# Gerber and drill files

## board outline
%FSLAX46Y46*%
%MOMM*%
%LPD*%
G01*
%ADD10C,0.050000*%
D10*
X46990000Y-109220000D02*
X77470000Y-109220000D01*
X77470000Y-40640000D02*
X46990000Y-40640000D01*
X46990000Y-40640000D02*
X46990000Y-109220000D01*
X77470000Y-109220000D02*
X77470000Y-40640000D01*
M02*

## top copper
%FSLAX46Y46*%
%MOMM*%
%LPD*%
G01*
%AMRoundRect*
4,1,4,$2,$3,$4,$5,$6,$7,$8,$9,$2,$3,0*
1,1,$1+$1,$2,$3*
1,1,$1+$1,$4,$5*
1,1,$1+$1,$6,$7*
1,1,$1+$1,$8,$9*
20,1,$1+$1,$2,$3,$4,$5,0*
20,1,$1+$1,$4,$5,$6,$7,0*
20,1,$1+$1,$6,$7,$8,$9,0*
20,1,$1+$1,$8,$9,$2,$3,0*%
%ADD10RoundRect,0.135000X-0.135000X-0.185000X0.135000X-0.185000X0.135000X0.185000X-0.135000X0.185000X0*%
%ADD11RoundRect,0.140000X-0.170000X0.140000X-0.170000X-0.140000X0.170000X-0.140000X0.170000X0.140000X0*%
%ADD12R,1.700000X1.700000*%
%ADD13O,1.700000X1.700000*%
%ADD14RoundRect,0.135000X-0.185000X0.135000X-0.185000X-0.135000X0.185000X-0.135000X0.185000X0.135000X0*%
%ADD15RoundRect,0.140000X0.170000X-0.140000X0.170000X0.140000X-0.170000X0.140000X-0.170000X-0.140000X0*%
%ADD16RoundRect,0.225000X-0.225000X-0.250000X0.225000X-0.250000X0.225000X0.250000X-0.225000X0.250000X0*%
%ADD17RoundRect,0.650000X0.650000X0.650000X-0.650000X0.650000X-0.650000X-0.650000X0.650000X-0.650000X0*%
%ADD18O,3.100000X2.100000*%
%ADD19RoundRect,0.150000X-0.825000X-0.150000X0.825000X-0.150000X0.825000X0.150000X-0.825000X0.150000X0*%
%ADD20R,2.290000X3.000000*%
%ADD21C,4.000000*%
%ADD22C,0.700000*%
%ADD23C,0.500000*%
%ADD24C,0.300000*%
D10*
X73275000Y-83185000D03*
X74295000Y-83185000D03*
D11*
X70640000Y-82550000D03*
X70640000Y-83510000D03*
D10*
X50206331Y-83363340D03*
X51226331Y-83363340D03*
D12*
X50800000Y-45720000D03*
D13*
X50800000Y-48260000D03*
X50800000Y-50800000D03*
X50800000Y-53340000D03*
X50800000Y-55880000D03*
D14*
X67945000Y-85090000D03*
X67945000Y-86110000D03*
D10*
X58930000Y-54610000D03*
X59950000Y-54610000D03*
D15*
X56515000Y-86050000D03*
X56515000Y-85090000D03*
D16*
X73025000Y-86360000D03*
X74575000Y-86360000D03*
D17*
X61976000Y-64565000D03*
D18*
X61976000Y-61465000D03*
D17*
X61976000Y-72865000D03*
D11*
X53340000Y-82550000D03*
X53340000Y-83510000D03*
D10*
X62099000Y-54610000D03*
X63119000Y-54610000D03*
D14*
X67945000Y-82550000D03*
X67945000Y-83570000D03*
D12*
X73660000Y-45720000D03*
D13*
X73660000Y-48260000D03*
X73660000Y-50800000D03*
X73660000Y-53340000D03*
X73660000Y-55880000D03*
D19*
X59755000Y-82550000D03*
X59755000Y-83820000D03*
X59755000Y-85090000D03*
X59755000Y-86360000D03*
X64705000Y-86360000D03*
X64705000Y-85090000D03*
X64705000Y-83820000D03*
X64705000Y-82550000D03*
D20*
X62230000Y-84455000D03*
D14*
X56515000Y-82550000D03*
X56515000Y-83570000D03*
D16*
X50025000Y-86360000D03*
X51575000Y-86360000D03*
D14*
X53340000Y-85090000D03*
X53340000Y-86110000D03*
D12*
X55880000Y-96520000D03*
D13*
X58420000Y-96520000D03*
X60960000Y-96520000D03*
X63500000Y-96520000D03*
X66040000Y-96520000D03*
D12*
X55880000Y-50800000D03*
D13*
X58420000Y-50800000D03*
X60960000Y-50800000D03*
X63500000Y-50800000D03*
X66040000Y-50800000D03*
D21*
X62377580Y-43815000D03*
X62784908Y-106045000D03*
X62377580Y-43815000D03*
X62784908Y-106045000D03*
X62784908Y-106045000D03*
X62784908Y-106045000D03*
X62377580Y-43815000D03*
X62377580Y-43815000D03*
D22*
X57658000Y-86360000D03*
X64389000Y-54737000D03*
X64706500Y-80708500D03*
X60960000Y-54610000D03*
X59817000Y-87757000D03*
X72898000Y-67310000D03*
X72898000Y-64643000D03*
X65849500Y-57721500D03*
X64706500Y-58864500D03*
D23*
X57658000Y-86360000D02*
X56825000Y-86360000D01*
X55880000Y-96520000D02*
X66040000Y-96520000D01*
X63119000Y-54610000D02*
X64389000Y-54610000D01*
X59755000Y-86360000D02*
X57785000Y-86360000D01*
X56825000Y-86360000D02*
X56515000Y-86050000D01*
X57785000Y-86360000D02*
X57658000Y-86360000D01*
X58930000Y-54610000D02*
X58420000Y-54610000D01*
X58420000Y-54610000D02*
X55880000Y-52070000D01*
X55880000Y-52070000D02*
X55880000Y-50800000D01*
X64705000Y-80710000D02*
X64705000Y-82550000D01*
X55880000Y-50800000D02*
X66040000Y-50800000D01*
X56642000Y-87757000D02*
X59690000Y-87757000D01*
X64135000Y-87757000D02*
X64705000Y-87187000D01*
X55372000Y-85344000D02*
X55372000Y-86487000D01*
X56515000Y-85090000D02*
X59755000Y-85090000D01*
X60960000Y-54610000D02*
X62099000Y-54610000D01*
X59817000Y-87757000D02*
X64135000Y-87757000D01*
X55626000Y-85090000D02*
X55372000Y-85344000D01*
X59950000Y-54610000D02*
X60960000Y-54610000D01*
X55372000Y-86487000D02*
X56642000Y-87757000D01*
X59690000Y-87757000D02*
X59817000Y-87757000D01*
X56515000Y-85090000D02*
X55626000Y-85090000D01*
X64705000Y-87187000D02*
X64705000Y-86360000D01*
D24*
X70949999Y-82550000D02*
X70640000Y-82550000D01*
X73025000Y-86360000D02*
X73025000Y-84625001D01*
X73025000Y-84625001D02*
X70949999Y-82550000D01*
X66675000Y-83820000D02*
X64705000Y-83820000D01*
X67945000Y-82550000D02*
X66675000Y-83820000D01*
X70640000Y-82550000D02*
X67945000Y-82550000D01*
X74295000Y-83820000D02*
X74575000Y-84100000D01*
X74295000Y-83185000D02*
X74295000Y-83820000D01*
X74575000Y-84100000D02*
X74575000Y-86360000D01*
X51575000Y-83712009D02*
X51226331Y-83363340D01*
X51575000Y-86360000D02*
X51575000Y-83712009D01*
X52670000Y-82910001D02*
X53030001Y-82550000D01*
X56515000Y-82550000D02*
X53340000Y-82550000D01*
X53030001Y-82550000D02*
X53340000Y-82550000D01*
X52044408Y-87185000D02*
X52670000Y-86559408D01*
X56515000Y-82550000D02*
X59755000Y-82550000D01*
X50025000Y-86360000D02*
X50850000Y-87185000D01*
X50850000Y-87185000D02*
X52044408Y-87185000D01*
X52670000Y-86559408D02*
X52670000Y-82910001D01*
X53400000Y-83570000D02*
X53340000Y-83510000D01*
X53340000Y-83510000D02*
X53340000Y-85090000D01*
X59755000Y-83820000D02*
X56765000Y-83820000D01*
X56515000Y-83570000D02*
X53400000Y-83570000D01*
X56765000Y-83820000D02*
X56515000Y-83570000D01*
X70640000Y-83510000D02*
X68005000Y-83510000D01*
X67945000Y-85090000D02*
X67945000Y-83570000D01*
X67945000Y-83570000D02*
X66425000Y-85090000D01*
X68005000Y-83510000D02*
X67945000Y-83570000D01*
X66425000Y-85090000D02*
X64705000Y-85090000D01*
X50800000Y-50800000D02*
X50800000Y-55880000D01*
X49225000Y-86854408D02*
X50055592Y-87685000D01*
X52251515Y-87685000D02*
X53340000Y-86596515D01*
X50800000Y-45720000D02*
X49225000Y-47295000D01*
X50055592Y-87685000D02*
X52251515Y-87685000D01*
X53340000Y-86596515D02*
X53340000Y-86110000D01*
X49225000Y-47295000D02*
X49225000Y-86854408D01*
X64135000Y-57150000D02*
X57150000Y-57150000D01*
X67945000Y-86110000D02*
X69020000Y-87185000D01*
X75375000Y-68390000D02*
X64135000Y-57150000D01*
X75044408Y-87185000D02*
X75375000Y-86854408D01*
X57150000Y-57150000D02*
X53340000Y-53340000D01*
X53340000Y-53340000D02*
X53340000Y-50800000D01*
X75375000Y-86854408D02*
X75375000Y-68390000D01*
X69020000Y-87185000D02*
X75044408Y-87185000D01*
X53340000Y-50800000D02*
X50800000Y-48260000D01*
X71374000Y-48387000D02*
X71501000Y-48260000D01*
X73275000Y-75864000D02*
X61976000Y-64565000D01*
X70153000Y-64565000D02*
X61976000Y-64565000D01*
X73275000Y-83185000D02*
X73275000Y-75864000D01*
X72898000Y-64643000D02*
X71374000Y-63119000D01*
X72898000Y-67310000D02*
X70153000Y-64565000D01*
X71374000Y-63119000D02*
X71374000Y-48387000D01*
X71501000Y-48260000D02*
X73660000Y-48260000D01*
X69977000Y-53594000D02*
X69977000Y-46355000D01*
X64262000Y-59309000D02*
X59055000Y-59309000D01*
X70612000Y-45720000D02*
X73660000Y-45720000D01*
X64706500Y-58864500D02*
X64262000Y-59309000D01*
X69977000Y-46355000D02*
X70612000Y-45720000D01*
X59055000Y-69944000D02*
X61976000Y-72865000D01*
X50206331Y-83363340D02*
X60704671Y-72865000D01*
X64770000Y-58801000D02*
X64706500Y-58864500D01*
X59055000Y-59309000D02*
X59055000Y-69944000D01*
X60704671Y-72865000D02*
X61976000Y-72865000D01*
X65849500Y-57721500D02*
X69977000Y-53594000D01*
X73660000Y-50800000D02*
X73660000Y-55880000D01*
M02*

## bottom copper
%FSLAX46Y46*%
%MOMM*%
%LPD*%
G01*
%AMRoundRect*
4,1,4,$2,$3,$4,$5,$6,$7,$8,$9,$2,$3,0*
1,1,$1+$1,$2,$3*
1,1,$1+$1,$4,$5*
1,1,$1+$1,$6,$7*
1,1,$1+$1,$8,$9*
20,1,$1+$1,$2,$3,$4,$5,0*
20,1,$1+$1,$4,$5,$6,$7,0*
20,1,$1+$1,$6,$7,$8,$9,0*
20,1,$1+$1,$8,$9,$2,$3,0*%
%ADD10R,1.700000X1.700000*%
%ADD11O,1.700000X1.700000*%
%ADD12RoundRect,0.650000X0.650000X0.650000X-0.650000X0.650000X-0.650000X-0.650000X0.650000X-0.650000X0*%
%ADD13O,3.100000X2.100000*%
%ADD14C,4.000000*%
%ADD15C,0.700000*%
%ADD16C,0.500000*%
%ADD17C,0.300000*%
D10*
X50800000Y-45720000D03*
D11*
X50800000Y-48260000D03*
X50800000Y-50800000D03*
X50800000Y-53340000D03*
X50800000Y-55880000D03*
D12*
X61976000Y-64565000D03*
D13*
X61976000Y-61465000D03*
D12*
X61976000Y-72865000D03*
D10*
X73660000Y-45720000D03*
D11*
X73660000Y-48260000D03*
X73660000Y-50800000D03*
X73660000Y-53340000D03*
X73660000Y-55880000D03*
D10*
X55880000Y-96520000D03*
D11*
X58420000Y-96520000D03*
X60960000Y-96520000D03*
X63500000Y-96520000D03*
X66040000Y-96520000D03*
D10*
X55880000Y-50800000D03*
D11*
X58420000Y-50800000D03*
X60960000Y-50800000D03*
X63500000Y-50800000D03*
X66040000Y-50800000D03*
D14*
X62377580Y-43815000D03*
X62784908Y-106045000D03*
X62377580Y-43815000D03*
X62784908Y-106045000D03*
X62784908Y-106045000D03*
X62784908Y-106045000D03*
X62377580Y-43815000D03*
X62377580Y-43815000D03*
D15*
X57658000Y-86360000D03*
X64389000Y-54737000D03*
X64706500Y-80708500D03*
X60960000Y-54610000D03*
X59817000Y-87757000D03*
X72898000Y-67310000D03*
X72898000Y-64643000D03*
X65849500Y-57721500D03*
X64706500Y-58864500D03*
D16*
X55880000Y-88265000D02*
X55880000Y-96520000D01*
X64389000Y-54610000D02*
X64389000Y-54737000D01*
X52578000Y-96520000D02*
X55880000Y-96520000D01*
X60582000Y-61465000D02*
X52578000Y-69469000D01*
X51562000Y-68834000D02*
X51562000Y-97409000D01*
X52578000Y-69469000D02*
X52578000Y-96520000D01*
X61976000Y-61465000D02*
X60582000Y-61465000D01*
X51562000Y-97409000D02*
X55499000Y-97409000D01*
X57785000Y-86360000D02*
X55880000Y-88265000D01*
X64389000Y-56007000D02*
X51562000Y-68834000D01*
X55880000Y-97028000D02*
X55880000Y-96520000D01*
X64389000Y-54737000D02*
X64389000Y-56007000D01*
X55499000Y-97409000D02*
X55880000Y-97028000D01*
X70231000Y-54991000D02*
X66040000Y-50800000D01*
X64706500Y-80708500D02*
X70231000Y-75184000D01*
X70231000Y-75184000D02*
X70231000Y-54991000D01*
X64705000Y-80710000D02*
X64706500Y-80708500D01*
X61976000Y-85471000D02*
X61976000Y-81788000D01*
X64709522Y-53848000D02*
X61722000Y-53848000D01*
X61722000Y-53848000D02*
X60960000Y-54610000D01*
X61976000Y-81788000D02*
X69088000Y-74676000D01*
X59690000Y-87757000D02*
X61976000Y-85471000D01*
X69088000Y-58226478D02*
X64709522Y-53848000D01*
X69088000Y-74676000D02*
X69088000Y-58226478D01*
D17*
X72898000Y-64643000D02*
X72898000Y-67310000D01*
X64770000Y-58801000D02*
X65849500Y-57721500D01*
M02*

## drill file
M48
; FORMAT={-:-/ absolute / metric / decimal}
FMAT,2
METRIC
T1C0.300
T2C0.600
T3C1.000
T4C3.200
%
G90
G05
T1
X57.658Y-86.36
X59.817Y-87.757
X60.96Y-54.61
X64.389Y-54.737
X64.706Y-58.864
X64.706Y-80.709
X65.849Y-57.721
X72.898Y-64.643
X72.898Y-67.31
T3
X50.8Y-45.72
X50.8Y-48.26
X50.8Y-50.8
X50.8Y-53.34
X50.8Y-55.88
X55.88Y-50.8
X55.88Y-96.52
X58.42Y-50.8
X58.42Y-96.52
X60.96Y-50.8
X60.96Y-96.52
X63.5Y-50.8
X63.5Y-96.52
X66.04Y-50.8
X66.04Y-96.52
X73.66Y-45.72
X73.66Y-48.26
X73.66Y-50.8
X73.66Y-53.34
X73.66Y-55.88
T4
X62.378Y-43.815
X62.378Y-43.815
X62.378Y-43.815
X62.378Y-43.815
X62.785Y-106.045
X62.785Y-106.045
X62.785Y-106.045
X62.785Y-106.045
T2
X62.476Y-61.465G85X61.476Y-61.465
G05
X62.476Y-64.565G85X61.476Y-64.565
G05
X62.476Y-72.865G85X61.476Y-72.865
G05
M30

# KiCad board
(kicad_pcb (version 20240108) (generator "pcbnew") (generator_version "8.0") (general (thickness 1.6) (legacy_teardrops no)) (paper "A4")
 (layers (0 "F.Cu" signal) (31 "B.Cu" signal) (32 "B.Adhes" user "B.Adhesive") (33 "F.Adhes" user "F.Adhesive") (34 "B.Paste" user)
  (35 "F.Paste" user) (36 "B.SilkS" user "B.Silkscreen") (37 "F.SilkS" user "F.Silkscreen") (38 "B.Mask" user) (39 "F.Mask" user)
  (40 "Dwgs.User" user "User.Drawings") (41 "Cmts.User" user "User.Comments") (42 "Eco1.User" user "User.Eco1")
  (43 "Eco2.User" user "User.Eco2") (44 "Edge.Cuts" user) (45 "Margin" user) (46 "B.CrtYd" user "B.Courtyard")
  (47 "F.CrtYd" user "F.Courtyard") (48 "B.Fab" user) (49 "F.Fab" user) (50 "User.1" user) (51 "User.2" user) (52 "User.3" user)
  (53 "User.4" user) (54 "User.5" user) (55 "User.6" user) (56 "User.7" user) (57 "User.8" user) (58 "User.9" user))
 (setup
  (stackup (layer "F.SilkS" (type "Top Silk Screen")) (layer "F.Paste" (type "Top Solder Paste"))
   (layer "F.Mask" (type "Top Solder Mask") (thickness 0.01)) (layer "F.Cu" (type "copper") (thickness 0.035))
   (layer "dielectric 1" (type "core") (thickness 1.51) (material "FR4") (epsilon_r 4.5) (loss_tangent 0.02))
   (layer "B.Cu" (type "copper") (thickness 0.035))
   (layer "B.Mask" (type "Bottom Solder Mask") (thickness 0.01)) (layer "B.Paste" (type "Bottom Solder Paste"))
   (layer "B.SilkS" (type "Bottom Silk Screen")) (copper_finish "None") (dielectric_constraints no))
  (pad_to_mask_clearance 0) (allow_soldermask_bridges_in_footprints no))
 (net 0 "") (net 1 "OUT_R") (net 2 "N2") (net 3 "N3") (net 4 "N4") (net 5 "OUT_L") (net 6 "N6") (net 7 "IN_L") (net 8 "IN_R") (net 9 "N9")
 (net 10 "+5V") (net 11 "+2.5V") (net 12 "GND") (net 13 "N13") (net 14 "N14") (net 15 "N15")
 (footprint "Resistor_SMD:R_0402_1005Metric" (layer "F.Cu") (at 73.785 83.185)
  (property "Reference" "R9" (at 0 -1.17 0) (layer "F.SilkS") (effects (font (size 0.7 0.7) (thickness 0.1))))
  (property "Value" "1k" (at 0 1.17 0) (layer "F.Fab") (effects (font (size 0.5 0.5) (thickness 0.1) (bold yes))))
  (pad "1" smd roundrect (at -0.51 0) (size 0.54 0.64) (layers "F.Cu" "F.Paste" "F.Mask") (roundrect_rratio 0.25) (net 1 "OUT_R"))
  (pad "2" smd roundrect (at 0.51 0) (size 0.54 0.64) (layers "F.Cu" "F.Paste" "F.Mask") (roundrect_rratio 0.25) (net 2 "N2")))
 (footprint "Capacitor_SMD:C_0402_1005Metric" (layer "F.Cu") (at 70.64 83.03 -90)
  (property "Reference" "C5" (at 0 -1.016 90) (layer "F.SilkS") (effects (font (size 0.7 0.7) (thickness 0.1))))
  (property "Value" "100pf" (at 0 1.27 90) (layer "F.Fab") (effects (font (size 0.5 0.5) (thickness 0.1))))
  (pad "1" smd roundrect (at -0.48 0 270) (size 0.56 0.62) (layers "F.Cu" "F.Paste" "F.Mask") (roundrect_rratio 0.25) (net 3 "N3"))
  (pad "2" smd roundrect (at 0.48 0 270) (size 0.56 0.62) (layers "F.Cu" "F.Paste" "F.Mask") (roundrect_rratio 0.25) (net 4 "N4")))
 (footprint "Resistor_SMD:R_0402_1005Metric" (layer "F.Cu") (at 50.716331 83.36334)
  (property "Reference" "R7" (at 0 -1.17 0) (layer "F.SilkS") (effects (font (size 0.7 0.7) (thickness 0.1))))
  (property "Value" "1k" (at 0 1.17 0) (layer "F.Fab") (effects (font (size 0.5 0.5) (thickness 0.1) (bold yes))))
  (pad "1" smd roundrect (at -0.51 0) (size 0.54 0.64) (layers "F.Cu" "F.Paste" "F.Mask") (roundrect_rratio 0.25) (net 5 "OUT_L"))
  (pad "2" smd roundrect (at 0.51 0) (size 0.54 0.64) (layers "F.Cu" "F.Paste" "F.Mask") (roundrect_rratio 0.25) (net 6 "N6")))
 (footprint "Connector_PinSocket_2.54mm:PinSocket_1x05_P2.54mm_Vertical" (layer "F.Cu") (at 50.8 45.72)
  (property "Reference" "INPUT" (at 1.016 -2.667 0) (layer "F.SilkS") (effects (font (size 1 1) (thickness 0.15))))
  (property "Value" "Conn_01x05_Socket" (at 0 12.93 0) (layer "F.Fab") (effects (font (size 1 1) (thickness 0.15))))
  (pad "1" thru_hole rect (at 0 0) (size 1.7 1.7) (drill 1) (layers "*.Cu" "*.Mask") (remove_unused_layers no) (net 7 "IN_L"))
  (pad "2" thru_hole oval (at 0 2.54) (size 1.7 1.7) (drill 1) (layers "*.Cu" "*.Mask") (remove_unused_layers no) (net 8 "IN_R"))
  (pad "3" thru_hole oval (at 0 5.08) (size 1.7 1.7) (drill 1) (layers "*.Cu" "*.Mask") (remove_unused_layers no) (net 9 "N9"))
  (pad "4" thru_hole oval (at 0 7.62) (size 1.7 1.7) (drill 1) (layers "*.Cu" "*.Mask") (remove_unused_layers no) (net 9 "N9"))
  (pad "5" thru_hole oval (at 0 10.16) (size 1.7 1.7) (drill 1) (layers "*.Cu" "*.Mask") (remove_unused_layers no) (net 9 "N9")))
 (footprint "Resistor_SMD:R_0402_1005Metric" (layer "F.Cu") (at 67.945 85.6 -90)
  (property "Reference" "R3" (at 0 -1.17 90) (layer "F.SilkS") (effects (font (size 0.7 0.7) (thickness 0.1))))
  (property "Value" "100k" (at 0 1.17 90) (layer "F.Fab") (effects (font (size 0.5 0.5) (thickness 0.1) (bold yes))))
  (pad "1" smd roundrect (at -0.51 0 270) (size 0.54 0.64) (layers "F.Cu" "F.Paste" "F.Mask") (roundrect_rratio 0.25) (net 4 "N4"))
  (pad "2" smd roundrect (at 0.51 0 270) (size 0.54 0.64) (layers "F.Cu" "F.Paste" "F.Mask") (roundrect_rratio 0.25) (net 8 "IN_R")))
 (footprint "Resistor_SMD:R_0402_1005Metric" (layer "F.Cu") (at 59.44 54.61)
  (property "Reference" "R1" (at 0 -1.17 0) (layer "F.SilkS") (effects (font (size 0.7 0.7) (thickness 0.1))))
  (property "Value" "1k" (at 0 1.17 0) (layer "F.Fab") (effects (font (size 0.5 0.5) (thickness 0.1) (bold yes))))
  (pad "1" smd roundrect (at -0.51 0) (size 0.54 0.64) (layers "F.Cu" "F.Paste" "F.Mask") (roundrect_rratio 0.25) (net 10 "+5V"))
  (pad "2" smd roundrect (at 0.51 0) (size 0.54 0.64) (layers "F.Cu" "F.Paste" "F.Mask") (roundrect_rratio 0.25) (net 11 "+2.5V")))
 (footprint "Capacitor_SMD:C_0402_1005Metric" (layer "F.Cu") (at 56.515 85.57 90)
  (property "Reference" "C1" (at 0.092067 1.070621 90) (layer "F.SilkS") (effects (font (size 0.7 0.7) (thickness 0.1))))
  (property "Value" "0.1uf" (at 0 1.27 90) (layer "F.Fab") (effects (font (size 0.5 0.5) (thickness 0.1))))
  (pad "1" smd roundrect (at -0.48 0 90) (size 0.56 0.62) (layers "F.Cu" "F.Paste" "F.Mask") (roundrect_rratio 0.25) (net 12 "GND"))
  (pad "2" smd roundrect (at 0.48 0 90) (size 0.56 0.62) (layers "F.Cu" "F.Paste" "F.Mask") (roundrect_rratio 0.25) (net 11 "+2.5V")))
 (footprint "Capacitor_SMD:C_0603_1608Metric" (layer "F.Cu") (at 73.8 86.36)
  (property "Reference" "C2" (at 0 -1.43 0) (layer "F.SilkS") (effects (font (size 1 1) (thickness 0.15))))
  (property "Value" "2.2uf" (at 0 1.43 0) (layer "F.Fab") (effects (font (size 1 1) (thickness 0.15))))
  (pad "1" smd roundrect (at -0.775 0) (size 0.9 0.95) (layers "F.Cu" "F.Paste" "F.Mask") (roundrect_rratio 0.25) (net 3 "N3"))
  (pad "2" smd roundrect (at 0.775 0) (size 0.9 0.95) (layers "F.Cu" "F.Paste" "F.Mask") (roundrect_rratio 0.25) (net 2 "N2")))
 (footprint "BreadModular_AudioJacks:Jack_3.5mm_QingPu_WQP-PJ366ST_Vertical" (layer "F.Cu") (at 61.976 67.945 180)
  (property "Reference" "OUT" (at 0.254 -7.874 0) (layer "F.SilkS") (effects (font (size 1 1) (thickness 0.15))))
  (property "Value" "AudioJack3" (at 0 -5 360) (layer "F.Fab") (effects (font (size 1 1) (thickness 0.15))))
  (pad "R" thru_hole roundrect (at 0 3.38 180) (size 2.6 2.6) (drill oval 1.6 0.6) (layers "*.Cu" "*.Mask") (remove_unused_layers no)
   (roundrect_rratio 0.25) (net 1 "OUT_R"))
  (pad "S" thru_hole oval (at 0 6.48 180) (size 3.1 2.1) (drill oval 1.6 0.6) (layers "*.Cu" "*.Mask") (remove_unused_layers no)
   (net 12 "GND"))
  (pad "T" thru_hole roundrect (at 0 -4.92 180) (size 2.6 2.6) (drill oval 1.6 0.6) (layers "*.Cu" "*.Mask") (remove_unused_layers no)
   (roundrect_rratio 0.25) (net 5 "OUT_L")))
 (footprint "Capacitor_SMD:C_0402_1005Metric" (layer "F.Cu") (at 53.34 83.03 -90)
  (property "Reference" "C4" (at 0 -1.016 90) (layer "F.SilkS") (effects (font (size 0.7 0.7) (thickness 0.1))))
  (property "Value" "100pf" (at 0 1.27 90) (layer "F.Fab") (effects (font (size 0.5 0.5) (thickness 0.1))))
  (pad "1" smd roundrect (at -0.48 0 270) (size 0.56 0.62) (layers "F.Cu" "F.Paste" "F.Mask") (roundrect_rratio 0.25) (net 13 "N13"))
  (pad "2" smd roundrect (at 0.48 0 270) (size 0.56 0.62) (layers "F.Cu" "F.Paste" "F.Mask") (roundrect_rratio 0.25) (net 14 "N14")))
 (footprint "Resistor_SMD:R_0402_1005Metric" (layer "F.Cu") (at 62.609 54.61)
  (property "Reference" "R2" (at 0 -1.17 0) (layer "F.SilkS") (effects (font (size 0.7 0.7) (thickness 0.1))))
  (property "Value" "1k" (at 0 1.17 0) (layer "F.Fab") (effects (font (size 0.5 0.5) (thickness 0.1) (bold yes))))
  (pad "1" smd roundrect (at -0.51 0) (size 0.54 0.64) (layers "F.Cu" "F.Paste" "F.Mask") (roundrect_rratio 0.25) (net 11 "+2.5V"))
  (pad "2" smd roundrect (at 0.51 0) (size 0.54 0.64) (layers "F.Cu" "F.Paste" "F.Mask") (roundrect_rratio 0.25) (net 12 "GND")))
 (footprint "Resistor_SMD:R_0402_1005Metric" (layer "F.Cu") (at 67.945 83.06 -90)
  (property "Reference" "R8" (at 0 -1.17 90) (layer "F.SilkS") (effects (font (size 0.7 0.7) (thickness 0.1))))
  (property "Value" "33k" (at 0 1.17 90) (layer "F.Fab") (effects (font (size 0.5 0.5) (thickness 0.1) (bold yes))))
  (pad "1" smd roundrect (at -0.51 0 270) (size 0.54 0.64) (layers "F.Cu" "F.Paste" "F.Mask") (roundrect_rratio 0.25) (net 3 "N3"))
  (pad "2" smd roundrect (at 0.51 0 270) (size 0.54 0.64) (layers "F.Cu" "F.Paste" "F.Mask") (roundrect_rratio 0.25) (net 4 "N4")))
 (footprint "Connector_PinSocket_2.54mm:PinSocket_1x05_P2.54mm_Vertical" (layer "F.Cu") (at 73.66 45.72)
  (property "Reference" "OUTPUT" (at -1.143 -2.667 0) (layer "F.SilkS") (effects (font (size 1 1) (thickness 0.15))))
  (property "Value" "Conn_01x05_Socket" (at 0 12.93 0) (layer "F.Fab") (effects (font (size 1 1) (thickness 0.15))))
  (pad "1" thru_hole rect (at 0 0) (size 1.7 1.7) (drill 1) (layers "*.Cu" "*.Mask") (remove_unused_layers no) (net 5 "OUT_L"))
  (pad "2" thru_hole oval (at 0 2.54) (size 1.7 1.7) (drill 1) (layers "*.Cu" "*.Mask") (remove_unused_layers no) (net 1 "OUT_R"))
  (pad "3" thru_hole oval (at 0 5.08) (size 1.7 1.7) (drill 1) (layers "*.Cu" "*.Mask") (remove_unused_layers no) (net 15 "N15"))
  (pad "4" thru_hole oval (at 0 7.62) (size 1.7 1.7) (drill 1) (layers "*.Cu" "*.Mask") (remove_unused_layers no) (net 15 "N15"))
  (pad "5" thru_hole oval (at 0 10.16) (size 1.7 1.7) (drill 1) (layers "*.Cu" "*.Mask") (remove_unused_layers no) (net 15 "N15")))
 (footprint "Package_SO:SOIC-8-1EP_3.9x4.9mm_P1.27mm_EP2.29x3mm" (layer "F.Cu") (at 62.23 84.455)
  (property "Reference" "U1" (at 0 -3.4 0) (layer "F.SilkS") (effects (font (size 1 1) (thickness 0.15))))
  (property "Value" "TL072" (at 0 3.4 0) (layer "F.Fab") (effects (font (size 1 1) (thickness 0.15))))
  (pad "" smd roundrect (at -0.57 -0.75) (size 0.92 1.21) (layers "F.Paste") (roundrect_rratio 0.25))
  (pad "" smd roundrect (at -0.57 0.75) (size 0.92 1.21) (layers "F.Paste") (roundrect_rratio 0.25))
  (pad "" smd roundrect (at 0.57 -0.75) (size 0.92 1.21) (layers "F.Paste") (roundrect_rratio 0.25))
  (pad "" smd roundrect (at 0.57 0.75) (size 0.92 1.21) (layers "F.Paste") (roundrect_rratio 0.25))
  (pad "1" smd roundrect (at -2.475 -1.905) (size 1.95 0.6) (layers "F.Cu" "F.Paste" "F.Mask") (roundrect_rratio 0.25) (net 13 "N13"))
  (pad "2" smd roundrect (at -2.475 -0.635) (size 1.95 0.6) (layers "F.Cu" "F.Paste" "F.Mask") (roundrect_rratio 0.25) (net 14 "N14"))
  (pad "3" smd roundrect (at -2.475 0.635) (size 1.95 0.6) (layers "F.Cu" "F.Paste" "F.Mask") (roundrect_rratio 0.25) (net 11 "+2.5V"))
  (pad "4" smd roundrect (at -2.475 1.905) (size 1.95 0.6) (layers "F.Cu" "F.Paste" "F.Mask") (roundrect_rratio 0.25) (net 12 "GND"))
  (pad "5" smd roundrect (at 2.475 1.905) (size 1.95 0.6) (layers "F.Cu" "F.Paste" "F.Mask") (roundrect_rratio 0.25) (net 11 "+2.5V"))
  (pad "6" smd roundrect (at 2.475 0.635) (size 1.95 0.6) (layers "F.Cu" "F.Paste" "F.Mask") (roundrect_rratio 0.25) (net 4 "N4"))
  (pad "7" smd roundrect (at 2.475 -0.635) (size 1.95 0.6) (layers "F.Cu" "F.Paste" "F.Mask") (roundrect_rratio 0.25) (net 3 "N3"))
  (pad "8" smd roundrect (at 2.475 -1.905) (size 1.95 0.6) (layers "F.Cu" "F.Paste" "F.Mask") (roundrect_rratio 0.25) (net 10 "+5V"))
  (pad "9" smd rect (at 0 0) (size 2.29 3) (layers "F.Cu" "F.Mask") (zone_connect 2)))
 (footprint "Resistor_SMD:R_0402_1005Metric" (layer "F.Cu") (at 56.515 83.06 -90)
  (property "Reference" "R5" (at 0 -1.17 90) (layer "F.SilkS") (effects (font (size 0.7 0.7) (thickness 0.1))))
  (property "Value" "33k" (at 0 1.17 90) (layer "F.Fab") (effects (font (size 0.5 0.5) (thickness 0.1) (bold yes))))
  (pad "1" smd roundrect (at -0.51 0 270) (size 0.54 0.64) (layers "F.Cu" "F.Paste" "F.Mask") (roundrect_rratio 0.25) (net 13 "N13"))
  (pad "2" smd roundrect (at 0.51 0 270) (size 0.54 0.64) (layers "F.Cu" "F.Paste" "F.Mask") (roundrect_rratio 0.25) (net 14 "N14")))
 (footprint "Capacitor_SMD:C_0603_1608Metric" (layer "F.Cu") (at 50.8 86.36)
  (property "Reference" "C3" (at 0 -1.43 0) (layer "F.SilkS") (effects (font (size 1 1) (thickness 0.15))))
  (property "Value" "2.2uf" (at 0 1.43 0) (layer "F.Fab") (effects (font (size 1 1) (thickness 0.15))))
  (pad "1" smd roundrect (at -0.775 0) (size 0.9 0.95) (layers "F.Cu" "F.Paste" "F.Mask") (roundrect_rratio 0.25) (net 13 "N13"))
  (pad "2" smd roundrect (at 0.775 0) (size 0.9 0.95) (layers "F.Cu" "F.Paste" "F.Mask") (roundrect_rratio 0.25) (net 6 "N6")))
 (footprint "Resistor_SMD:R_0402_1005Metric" (layer "F.Cu") (at 53.34 85.6 -90)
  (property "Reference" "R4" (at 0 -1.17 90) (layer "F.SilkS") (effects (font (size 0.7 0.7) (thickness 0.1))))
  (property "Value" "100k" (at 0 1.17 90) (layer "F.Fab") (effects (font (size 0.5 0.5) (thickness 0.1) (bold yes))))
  (pad "1" smd roundrect (at -0.51 0 270) (size 0.54 0.64) (layers "F.Cu" "F.Paste" "F.Mask") (roundrect_rratio 0.25) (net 14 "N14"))
  (pad "2" smd roundrect (at 0.51 0 270) (size 0.54 0.64) (layers "F.Cu" "F.Paste" "F.Mask") (roundrect_rratio 0.25) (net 7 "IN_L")))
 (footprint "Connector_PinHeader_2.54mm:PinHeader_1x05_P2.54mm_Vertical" (layer "B.Cu") (at 55.88 96.52 -90)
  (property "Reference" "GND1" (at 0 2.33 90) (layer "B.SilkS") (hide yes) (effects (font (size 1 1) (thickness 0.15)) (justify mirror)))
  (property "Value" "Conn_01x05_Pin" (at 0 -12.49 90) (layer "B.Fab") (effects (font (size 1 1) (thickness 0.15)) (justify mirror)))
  (pad "1" thru_hole rect (at 0 0 270) (size 1.7 1.7) (drill 1) (layers "*.Cu" "*.Mask") (remove_unused_layers no) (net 12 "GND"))
  (pad "2" thru_hole oval (at 0 -2.54 270) (size 1.7 1.7) (drill 1) (layers "*.Cu" "*.Mask") (remove_unused_layers no) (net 12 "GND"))
  (pad "3" thru_hole oval (at 0 -5.08 270) (size 1.7 1.7) (drill 1) (layers "*.Cu" "*.Mask") (remove_unused_layers no) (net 12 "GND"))
  (pad "4" thru_hole oval (at 0 -7.62 270) (size 1.7 1.7) (drill 1) (layers "*.Cu" "*.Mask") (remove_unused_layers no) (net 12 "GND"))
  (pad "5" thru_hole oval (at 0 -10.16 270) (size 1.7 1.7) (drill 1) (layers "*.Cu" "*.Mask") (remove_unused_layers no) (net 12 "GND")))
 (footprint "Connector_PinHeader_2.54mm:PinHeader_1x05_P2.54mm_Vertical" (layer "B.Cu") (at 55.88 50.8 -90)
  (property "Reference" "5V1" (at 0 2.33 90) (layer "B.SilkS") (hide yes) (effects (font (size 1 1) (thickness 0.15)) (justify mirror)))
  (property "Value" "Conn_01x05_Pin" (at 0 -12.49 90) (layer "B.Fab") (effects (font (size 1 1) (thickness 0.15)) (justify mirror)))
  (pad "1" thru_hole rect (at 0 0 270) (size 1.7 1.7) (drill 1) (layers "*.Cu" "*.Mask") (remove_unused_layers no) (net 10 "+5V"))
  (pad "2" thru_hole oval (at 0 -2.54 270) (size 1.7 1.7) (drill 1) (layers "*.Cu" "*.Mask") (remove_unused_layers no) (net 10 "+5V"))
  (pad "3" thru_hole oval (at 0 -5.08 270) (size 1.7 1.7) (drill 1) (layers "*.Cu" "*.Mask") (remove_unused_layers no) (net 10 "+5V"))
  (pad "4" thru_hole oval (at 0 -7.62 270) (size 1.7 1.7) (drill 1) (layers "*.Cu" "*.Mask") (remove_unused_layers no) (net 10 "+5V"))
  (pad "5" thru_hole oval (at 0 -10.16 270) (size 1.7 1.7) (drill 1) (layers "*.Cu" "*.Mask") (remove_unused_layers no) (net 10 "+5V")))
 (gr_line (start 46.99 109.22) (end 77.47 109.22) (stroke (width 0.05) (type default)) (layer "Edge.Cuts"))
 (gr_line (start 77.47 40.64) (end 46.99 40.64) (stroke (width 0.05) (type default)) (layer "Edge.Cuts"))
 (gr_line (start 46.99 40.64) (end 46.99 109.22) (stroke (width 0.05) (type default)) (layer "Edge.Cuts"))
 (gr_line (start 77.47 109.22) (end 77.47 40.64) (stroke (width 0.05) (type default)) (layer "Edge.Cuts"))
 (via (at 62.37758 43.815) (size 4) (drill 3.2) (layers "F.Cu" "B.Cu") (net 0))
 (via (at 62.784908 106.045) (size 4) (drill 3.2) (layers "F.Cu" "B.Cu") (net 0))
 (via (at 62.37758 43.815) (size 4) (drill 3.2) (layers "F.Cu" "B.Cu") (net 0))
 (via (at 62.784908 106.045) (size 4) (drill 3.2) (layers "F.Cu" "B.Cu") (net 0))
 (via (at 62.784908 106.045) (size 4) (drill 3.2) (layers "F.Cu" "B.Cu") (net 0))
 (via (at 62.784908 106.045) (size 4) (drill 3.2) (layers "F.Cu" "B.Cu") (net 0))
 (via (at 62.37758 43.815) (size 4) (drill 3.2) (layers "F.Cu" "B.Cu") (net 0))
 (via (at 62.37758 43.815) (size 4) (drill 3.2) (layers "F.Cu" "B.Cu") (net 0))
 (segment (start 57.658 86.36) (end 56.825 86.36) (width 0.5) (layer "F.Cu") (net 12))
 (segment (start 55.88 96.52) (end 66.04 96.52) (width 0.5) (layer "F.Cu") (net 12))
 (segment (start 63.119 54.61) (end 64.389 54.61) (width 0.5) (layer "F.Cu") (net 12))
 (segment (start 59.755 86.36) (end 57.785 86.36) (width 0.5) (layer "F.Cu") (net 12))
 (segment (start 56.825 86.36) (end 56.515 86.05) (width 0.5) (layer "F.Cu") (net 12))
 (segment (start 57.785 86.36) (end 57.658 86.36) (width 0.5) (layer "F.Cu") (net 12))
 (via (at 57.658 86.36) (size 0.7) (drill 0.3) (layers "F.Cu" "B.Cu") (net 12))
 (via (at 64.389 54.737) (size 0.7) (drill 0.3) (layers "F.Cu" "B.Cu") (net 12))
 (segment (start 55.88 88.265) (end 55.88 96.52) (width 0.5) (layer "B.Cu") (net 12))
 (segment (start 64.389 54.61) (end 64.389 54.737) (width 0.5) (layer "B.Cu") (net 12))
 (segment (start 52.578 96.52) (end 55.88 96.52) (width 0.5) (layer "B.Cu") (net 12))
 (segment (start 60.582 61.465) (end 52.578 69.469) (width 0.5) (layer "B.Cu") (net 12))
 (segment (start 51.562 68.834) (end 51.562 97.409) (width 0.5) (layer "B.Cu") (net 12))
 (segment (start 52.578 69.469) (end 52.578 96.52) (width 0.5) (layer "B.Cu") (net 12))
 (segment (start 61.976 61.465) (end 60.582 61.465) (width 0.5) (layer "B.Cu") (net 12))
 (segment (start 51.562 97.409) (end 55.499 97.409) (width 0.5) (layer "B.Cu") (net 12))
 (segment (start 57.785 86.36) (end 55.88 88.265) (width 0.5) (layer "B.Cu") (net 12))
 (segment (start 64.389 56.007) (end 51.562 68.834) (width 0.5) (layer "B.Cu") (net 12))
 (segment (start 55.88 97.028) (end 55.88 96.52) (width 0.5) (layer "B.Cu") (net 12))
 (segment (start 64.389 54.737) (end 64.389 56.007) (width 0.5) (layer "B.Cu") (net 12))
 (segment (start 55.499 97.409) (end 55.88 97.028) (width 0.5) (layer "B.Cu") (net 12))
 (segment (start 58.93 54.61) (end 58.42 54.61) (width 0.5) (layer "F.Cu") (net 10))
 (segment (start 58.42 54.61) (end 55.88 52.07) (width 0.5) (layer "F.Cu") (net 10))
 (segment (start 55.88 52.07) (end 55.88 50.8) (width 0.5) (layer "F.Cu") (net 10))
 (segment (start 64.705 80.71) (end 64.705 82.55) (width 0.5) (layer "F.Cu") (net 10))
 (segment (start 55.88 50.8) (end 66.04 50.8) (width 0.5) (layer "F.Cu") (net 10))
 (via (at 64.7065 80.7085) (size 0.7) (drill 0.3) (layers "F.Cu" "B.Cu") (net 10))
 (segment (start 70.231 54.991) (end 66.04 50.8) (width 0.5) (layer "B.Cu") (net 10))
 (segment (start 64.7065 80.7085) (end 70.231 75.184) (width 0.5) (layer "B.Cu") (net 10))
 (segment (start 70.231 75.184) (end 70.231 54.991) (width 0.5) (layer "B.Cu") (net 10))
 (segment (start 64.705 80.71) (end 64.7065 80.7085) (width 0.5) (layer "B.Cu") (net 10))
 (segment (start 56.642 87.757) (end 59.69 87.757) (width 0.5) (layer "F.Cu") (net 11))
 (segment (start 64.135 87.757) (end 64.705 87.187) (width 0.5) (layer "F.Cu") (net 11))
 (segment (start 55.372 85.344) (end 55.372 86.487) (width 0.5) (layer "F.Cu") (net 11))
 (segment (start 56.515 85.09) (end 59.755 85.09) (width 0.5) (layer "F.Cu") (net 11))
 (segment (start 60.96 54.61) (end 62.099 54.61) (width 0.5) (layer "F.Cu") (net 11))
 (segment (start 59.817 87.757) (end 64.135 87.757) (width 0.5) (layer "F.Cu") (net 11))
 (segment (start 55.626 85.09) (end 55.372 85.344) (width 0.5) (layer "F.Cu") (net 11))
 (segment (start 59.95 54.61) (end 60.96 54.61) (width 0.5) (layer "F.Cu") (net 11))
 (segment (start 55.372 86.487) (end 56.642 87.757) (width 0.5) (layer "F.Cu") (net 11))
 (segment (start 59.69 87.757) (end 59.817 87.757) (width 0.5) (layer "F.Cu") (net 11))
 (segment (start 56.515 85.09) (end 55.626 85.09) (width 0.5) (layer "F.Cu") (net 11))
 (segment (start 64.705 87.187) (end 64.705 86.36) (width 0.5) (layer "F.Cu") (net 11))
 (via (at 60.96 54.61) (size 0.7) (drill 0.3) (layers "F.Cu" "B.Cu") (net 11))
 (via (at 59.817 87.757) (size 0.7) (drill 0.3) (layers "F.Cu" "B.Cu") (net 11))
 (segment (start 61.976 85.471) (end 61.976 81.788) (width 0.5) (layer "B.Cu") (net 11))
 (segment (start 64.709522 53.848) (end 61.722 53.848) (width 0.5) (layer "B.Cu") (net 11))
 (segment (start 61.722 53.848) (end 60.96 54.61) (width 0.5) (layer "B.Cu") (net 11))
 (segment (start 61.976 81.788) (end 69.088 74.676) (width 0.5) (layer "B.Cu") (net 11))
 (segment (start 59.69 87.757) (end 61.976 85.471) (width 0.5) (layer "B.Cu") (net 11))
 (segment (start 69.088 58.226478) (end 64.709522 53.848) (width 0.5) (layer "B.Cu") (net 11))
 (segment (start 69.088 74.676) (end 69.088 58.226478) (width 0.5) (layer "B.Cu") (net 11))
 (segment (start 70.949999 82.55) (end 70.64 82.55) (width 0.3) (layer "F.Cu") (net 3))
 (segment (start 73.025 86.36) (end 73.025 84.625001) (width 0.3) (layer "F.Cu") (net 3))
 (segment (start 73.025 84.625001) (end 70.949999 82.55) (width 0.3) (layer "F.Cu") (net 3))
 (segment (start 66.675 83.82) (end 64.705 83.82) (width 0.3) (layer "F.Cu") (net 3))
 (segment (start 67.945 82.55) (end 66.675 83.82) (width 0.3) (layer "F.Cu") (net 3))
 (segment (start 70.64 82.55) (end 67.945 82.55) (width 0.3) (layer "F.Cu") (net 3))
 (segment (start 74.295 83.82) (end 74.575 84.1) (width 0.3) (layer "F.Cu") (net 2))
 (segment (start 74.295 83.185) (end 74.295 83.82) (width 0.3) (layer "F.Cu") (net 2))
 (segment (start 74.575 84.1) (end 74.575 86.36) (width 0.3) (layer "F.Cu") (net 2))
 (segment (start 51.575 83.712009) (end 51.226331 83.36334) (width 0.3) (layer "F.Cu") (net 6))
 (segment (start 51.575 86.36) (end 51.575 83.712009) (width 0.3) (layer "F.Cu") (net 6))
 (segment (start 52.67 82.910001) (end 53.030001 82.55) (width 0.3) (layer "F.Cu") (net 13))
 (segment (start 56.515 82.55) (end 53.34 82.55) (width 0.3) (layer "F.Cu") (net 13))
 (segment (start 53.030001 82.55) (end 53.34 82.55) (width 0.3) (layer "F.Cu") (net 13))
 (segment (start 52.044408 87.185) (end 52.67 86.559408) (width 0.3) (layer "F.Cu") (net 13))
 (segment (start 56.515 82.55) (end 59.755 82.55) (width 0.3) (layer "F.Cu") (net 13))
 (segment (start 50.025 86.36) (end 50.85 87.185) (width 0.3) (layer "F.Cu") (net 13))
 (segment (start 50.85 87.185) (end 52.044408 87.185) (width 0.3) (layer "F.Cu") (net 13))
 (segment (start 52.67 86.559408) (end 52.67 82.910001) (width 0.3) (layer "F.Cu") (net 13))
 (segment (start 53.4 83.57) (end 53.34 83.51) (width 0.3) (layer "F.Cu") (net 14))
 (segment (start 53.34 83.51) (end 53.34 85.09) (width 0.3) (layer "F.Cu") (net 14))
 (segment (start 59.755 83.82) (end 56.765 83.82) (width 0.3) (layer "F.Cu") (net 14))
 (segment (start 56.515 83.57) (end 53.4 83.57) (width 0.3) (layer "F.Cu") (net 14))
 (segment (start 56.765 83.82) (end 56.515 83.57) (width 0.3) (layer "F.Cu") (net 14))
 (segment (start 70.64 83.51) (end 68.005 83.51) (width 0.3) (layer "F.Cu") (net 4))
 (segment (start 67.945 85.09) (end 67.945 83.57) (width 0.3) (layer "F.Cu") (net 4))
 (segment (start 67.945 83.57) (end 66.425 85.09) (width 0.3) (layer "F.Cu") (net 4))
 (segment (start 68.005 83.51) (end 67.945 83.57) (width 0.3) (layer "F.Cu") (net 4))
 (segment (start 66.425 85.09) (end 64.705 85.09) (width 0.3) (layer "F.Cu") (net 4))
 (segment (start 50.8 50.8) (end 50.8 55.88) (width 0.3) (layer "F.Cu") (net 9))
 (segment (start 49.225 86.854408) (end 50.055592 87.685) (width 0.3) (layer "F.Cu") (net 7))
 (segment (start 52.251515 87.685) (end 53.34 86.596515) (width 0.3) (layer "F.Cu") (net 7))
 (segment (start 50.8 45.72) (end 49.225 47.295) (width 0.3) (layer "F.Cu") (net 7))
 (segment (start 50.055592 87.685) (end 52.251515 87.685) (width 0.3) (layer "F.Cu") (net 7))
 (segment (start 53.34 86.596515) (end 53.34 86.11) (width 0.3) (layer "F.Cu") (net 7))
 (segment (start 49.225 47.295) (end 49.225 86.854408) (width 0.3) (layer "F.Cu") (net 7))
 (segment (start 64.135 57.15) (end 57.15 57.15) (width 0.3) (layer "F.Cu") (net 8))
 (segment (start 67.945 86.11) (end 69.02 87.185) (width 0.3) (layer "F.Cu") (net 8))
 (segment (start 75.375 68.39) (end 64.135 57.15) (width 0.3) (layer "F.Cu") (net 8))
 (segment (start 75.044408 87.185) (end 75.375 86.854408) (width 0.3) (layer "F.Cu") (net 8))
 (segment (start 57.15 57.15) (end 53.34 53.34) (width 0.3) (layer "F.Cu") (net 8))
 (segment (start 53.34 53.34) (end 53.34 50.8) (width 0.3) (layer "F.Cu") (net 8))
 (segment (start 75.375 86.854408) (end 75.375 68.39) (width 0.3) (layer "F.Cu") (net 8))
 (segment (start 69.02 87.185) (end 75.044408 87.185) (width 0.3) (layer "F.Cu") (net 8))
 (segment (start 53.34 50.8) (end 50.8 48.26) (width 0.3) (layer "F.Cu") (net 8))
 (segment (start 71.374 48.387) (end 71.501 48.26) (width 0.3) (layer "F.Cu") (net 1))
 (segment (start 73.275 75.864) (end 61.976 64.565) (width 0.3) (layer "F.Cu") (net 1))
 (segment (start 70.153 64.565) (end 61.976 64.565) (width 0.3) (layer "F.Cu") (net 1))
 (segment (start 73.275 83.185) (end 73.275 75.864) (width 0.3) (layer "F.Cu") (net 1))
 (segment (start 72.898 64.643) (end 71.374 63.119) (width 0.3) (layer "F.Cu") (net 1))
 (segment (start 72.898 67.31) (end 70.153 64.565) (width 0.3) (layer "F.Cu") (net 1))
 (segment (start 71.374 63.119) (end 71.374 48.387) (width 0.3) (layer "F.Cu") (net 1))
 (segment (start 71.501 48.26) (end 73.66 48.26) (width 0.3) (layer "F.Cu") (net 1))
 (via (at 72.898 67.31) (size 0.7) (drill 0.3) (layers "F.Cu" "B.Cu") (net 1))
 (via (at 72.898 64.643) (size 0.7) (drill 0.3) (layers "F.Cu" "B.Cu") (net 1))
 (segment (start 72.898 64.643) (end 72.898 67.31) (width 0.3) (layer "B.Cu") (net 1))
 (segment (start 69.977 53.594) (end 69.977 46.355) (width 0.3) (layer "F.Cu") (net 5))
 (segment (start 64.262 59.309) (end 59.055 59.309) (width 0.3) (layer "F.Cu") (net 5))
 (segment (start 70.612 45.72) (end 73.66 45.72) (width 0.3) (layer "F.Cu") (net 5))
 (segment (start 64.7065 58.8645) (end 64.262 59.309) (width 0.3) (layer "F.Cu") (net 5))
 (segment (start 69.977 46.355) (end 70.612 45.72) (width 0.3) (layer "F.Cu") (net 5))
 (segment (start 59.055 69.944) (end 61.976 72.865) (width 0.3) (layer "F.Cu") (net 5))
 (segment (start 50.206331 83.36334) (end 60.704671 72.865) (width 0.3) (layer "F.Cu") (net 5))
 (segment (start 64.77 58.801) (end 64.7065 58.8645) (width 0.3) (layer "F.Cu") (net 5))
 (segment (start 59.055 59.309) (end 59.055 69.944) (width 0.3) (layer "F.Cu") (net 5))
 (segment (start 60.704671 72.865) (end 61.976 72.865) (width 0.3) (layer "F.Cu") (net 5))
 (segment (start 65.8495 57.7215) (end 69.977 53.594) (width 0.3) (layer "F.Cu") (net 5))
 (via (at 65.8495 57.7215) (size 0.7) (drill 0.3) (layers "F.Cu" "B.Cu") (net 5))
 (via (at 64.7065 58.8645) (size 0.7) (drill 0.3) (layers "F.Cu" "B.Cu") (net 5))
 (segment (start 64.77 58.801) (end 65.8495 57.7215) (width 0.3) (layer "B.Cu") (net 5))
 (segment (start 73.66 50.8) (end 73.66 55.88) (width 0.3) (layer "F.Cu") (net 15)))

